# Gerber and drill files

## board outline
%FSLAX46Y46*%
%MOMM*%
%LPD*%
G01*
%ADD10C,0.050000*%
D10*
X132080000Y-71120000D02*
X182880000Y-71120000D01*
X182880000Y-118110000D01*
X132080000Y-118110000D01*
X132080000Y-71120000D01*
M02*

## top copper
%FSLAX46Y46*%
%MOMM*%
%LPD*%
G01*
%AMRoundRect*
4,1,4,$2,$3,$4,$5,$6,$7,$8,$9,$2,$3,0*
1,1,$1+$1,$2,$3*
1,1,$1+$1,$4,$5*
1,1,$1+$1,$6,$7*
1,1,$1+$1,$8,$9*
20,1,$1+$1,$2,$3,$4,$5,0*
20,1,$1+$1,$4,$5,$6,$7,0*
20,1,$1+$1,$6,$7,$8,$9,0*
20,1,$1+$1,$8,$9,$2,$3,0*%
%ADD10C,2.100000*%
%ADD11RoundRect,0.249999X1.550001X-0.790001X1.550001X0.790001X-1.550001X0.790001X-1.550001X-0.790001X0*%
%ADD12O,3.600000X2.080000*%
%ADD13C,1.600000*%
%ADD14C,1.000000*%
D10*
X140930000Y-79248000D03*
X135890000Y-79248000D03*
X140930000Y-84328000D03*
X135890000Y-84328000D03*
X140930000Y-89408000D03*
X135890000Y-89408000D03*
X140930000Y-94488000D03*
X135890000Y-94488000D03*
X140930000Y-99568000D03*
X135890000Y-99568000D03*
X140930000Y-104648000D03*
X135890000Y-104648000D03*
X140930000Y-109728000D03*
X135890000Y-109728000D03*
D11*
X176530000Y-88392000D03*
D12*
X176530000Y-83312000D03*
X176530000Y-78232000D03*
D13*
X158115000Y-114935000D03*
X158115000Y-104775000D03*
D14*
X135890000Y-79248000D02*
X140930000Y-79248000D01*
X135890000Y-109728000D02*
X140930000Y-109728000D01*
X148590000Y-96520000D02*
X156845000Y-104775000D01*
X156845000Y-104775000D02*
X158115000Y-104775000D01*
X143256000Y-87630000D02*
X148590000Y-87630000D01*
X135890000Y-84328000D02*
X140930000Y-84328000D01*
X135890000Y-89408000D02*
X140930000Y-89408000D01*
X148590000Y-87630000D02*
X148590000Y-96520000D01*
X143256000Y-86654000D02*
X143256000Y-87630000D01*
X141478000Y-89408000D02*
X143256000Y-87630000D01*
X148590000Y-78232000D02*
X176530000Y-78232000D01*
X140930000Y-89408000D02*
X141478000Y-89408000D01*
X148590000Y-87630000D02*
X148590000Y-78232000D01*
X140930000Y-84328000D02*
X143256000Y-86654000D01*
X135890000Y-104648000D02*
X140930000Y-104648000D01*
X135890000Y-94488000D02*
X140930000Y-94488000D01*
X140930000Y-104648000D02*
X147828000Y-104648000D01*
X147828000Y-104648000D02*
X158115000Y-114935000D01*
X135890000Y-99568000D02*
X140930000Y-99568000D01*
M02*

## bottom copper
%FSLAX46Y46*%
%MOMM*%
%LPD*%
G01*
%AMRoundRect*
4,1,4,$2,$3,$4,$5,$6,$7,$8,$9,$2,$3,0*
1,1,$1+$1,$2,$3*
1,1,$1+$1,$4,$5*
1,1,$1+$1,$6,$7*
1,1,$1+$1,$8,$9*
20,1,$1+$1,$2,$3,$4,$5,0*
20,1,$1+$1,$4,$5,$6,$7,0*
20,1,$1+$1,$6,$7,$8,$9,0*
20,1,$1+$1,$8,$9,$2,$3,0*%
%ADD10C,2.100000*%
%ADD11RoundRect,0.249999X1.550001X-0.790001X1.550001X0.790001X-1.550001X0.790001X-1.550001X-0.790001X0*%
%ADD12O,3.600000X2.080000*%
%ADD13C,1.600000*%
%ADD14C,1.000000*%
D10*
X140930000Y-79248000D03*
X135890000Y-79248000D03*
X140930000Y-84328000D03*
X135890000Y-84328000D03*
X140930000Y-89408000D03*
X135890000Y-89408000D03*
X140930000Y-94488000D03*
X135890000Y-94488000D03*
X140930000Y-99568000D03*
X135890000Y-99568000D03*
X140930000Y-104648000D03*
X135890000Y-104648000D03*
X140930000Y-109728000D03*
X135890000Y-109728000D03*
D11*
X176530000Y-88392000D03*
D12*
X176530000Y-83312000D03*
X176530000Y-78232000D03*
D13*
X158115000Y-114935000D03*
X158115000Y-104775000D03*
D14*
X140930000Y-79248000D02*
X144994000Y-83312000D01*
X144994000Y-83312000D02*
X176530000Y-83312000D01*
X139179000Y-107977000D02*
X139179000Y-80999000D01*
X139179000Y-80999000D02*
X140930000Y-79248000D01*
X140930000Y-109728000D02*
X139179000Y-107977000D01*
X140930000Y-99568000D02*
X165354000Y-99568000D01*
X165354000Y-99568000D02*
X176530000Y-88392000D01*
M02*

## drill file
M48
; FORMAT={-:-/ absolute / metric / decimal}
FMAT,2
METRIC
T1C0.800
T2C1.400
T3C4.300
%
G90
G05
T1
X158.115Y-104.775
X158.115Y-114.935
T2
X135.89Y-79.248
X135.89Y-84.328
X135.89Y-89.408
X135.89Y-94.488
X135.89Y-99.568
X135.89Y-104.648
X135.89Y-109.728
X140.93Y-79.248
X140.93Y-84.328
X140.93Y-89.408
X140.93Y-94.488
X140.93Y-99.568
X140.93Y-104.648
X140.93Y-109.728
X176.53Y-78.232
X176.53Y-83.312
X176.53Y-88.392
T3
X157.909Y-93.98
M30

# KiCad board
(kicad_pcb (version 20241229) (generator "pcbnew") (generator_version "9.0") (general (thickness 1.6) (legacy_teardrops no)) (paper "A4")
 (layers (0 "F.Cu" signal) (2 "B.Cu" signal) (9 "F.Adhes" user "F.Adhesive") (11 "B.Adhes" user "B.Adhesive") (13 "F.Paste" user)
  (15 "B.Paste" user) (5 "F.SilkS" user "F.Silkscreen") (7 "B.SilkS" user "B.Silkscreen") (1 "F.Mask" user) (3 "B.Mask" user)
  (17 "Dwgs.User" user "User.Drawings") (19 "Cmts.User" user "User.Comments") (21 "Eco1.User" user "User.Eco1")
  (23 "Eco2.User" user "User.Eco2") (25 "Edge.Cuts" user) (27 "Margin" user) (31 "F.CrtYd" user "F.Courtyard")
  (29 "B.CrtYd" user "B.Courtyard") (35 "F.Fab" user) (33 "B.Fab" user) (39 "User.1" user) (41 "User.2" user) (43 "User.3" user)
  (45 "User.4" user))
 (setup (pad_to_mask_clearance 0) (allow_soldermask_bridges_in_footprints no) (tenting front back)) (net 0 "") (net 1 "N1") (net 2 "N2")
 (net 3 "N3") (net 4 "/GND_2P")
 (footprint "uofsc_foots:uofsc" (layer "F.Cu") (at 174.498 108.204)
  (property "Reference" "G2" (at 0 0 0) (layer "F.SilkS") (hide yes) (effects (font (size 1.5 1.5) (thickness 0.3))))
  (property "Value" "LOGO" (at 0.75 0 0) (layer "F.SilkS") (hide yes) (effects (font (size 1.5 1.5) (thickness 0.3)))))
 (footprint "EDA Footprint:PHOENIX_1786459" (layer "F.Cu") (at 124.76 75.708 -90)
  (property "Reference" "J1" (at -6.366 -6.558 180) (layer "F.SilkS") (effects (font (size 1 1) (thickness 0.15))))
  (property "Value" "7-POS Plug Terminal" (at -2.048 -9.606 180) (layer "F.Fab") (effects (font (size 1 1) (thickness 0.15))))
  (pad "1" thru_hole circle (at 3.54 -16.17 270) (size 2.1 2.1) (drill 1.4) (layers "*.Cu" "*.Mask") (remove_unused_layers no) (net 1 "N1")
   (solder_mask_margin 0.102))
  (pad "1" thru_hole circle (at 3.54 -11.13 270) (size 2.1 2.1) (drill 1.4) (layers "*.Cu" "*.Mask") (remove_unused_layers no) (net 1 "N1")
   (solder_mask_margin 0.102))
  (pad "2" thru_hole circle (at 8.62 -16.17 270) (size 2.1 2.1) (drill 1.4) (layers "*.Cu" "*.Mask") (remove_unused_layers no) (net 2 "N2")
   (solder_mask_margin 0.102))
  (pad "2" thru_hole circle (at 8.62 -11.13 270) (size 2.1 2.1) (drill 1.4) (layers "*.Cu" "*.Mask") (remove_unused_layers no) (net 2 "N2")
   (solder_mask_margin 0.102))
  (pad "3" thru_hole circle (at 13.7 -16.17 270) (size 2.1 2.1) (drill 1.4) (layers "*.Cu" "*.Mask") (remove_unused_layers no) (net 2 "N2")
   (solder_mask_margin 0.102))
  (pad "3" thru_hole circle (at 13.7 -11.13 270) (size 2.1 2.1) (drill 1.4) (layers "*.Cu" "*.Mask") (remove_unused_layers no) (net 2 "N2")
   (solder_mask_margin 0.102))
  (pad "4" thru_hole circle (at 18.78 -16.17 270) (size 2.1 2.1) (drill 1.4) (layers "*.Cu" "*.Mask") (remove_unused_layers no) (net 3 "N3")
   (solder_mask_margin 0.102))
  (pad "4" thru_hole circle (at 18.78 -11.13 270) (size 2.1 2.1) (drill 1.4) (layers "*.Cu" "*.Mask") (remove_unused_layers no) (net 3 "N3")
   (solder_mask_margin 0.102))
  (pad "5" thru_hole circle (at 23.86 -16.17 270) (size 2.1 2.1) (drill 1.4) (layers "*.Cu" "*.Mask") (remove_unused_layers no)
   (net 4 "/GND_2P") (solder_mask_margin 0.102))
  (pad "5" thru_hole circle (at 23.86 -11.13 270) (size 2.1 2.1) (drill 1.4) (layers "*.Cu" "*.Mask") (remove_unused_layers no)
   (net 4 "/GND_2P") (solder_mask_margin 0.102))
  (pad "6" thru_hole circle (at 28.94 -16.17 270) (size 2.1 2.1) (drill 1.4) (layers "*.Cu" "*.Mask") (remove_unused_layers no) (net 3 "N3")
   (solder_mask_margin 0.102))
  (pad "6" thru_hole circle (at 28.94 -11.13 270) (size 2.1 2.1) (drill 1.4) (layers "*.Cu" "*.Mask") (remove_unused_layers no) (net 3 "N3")
   (solder_mask_margin 0.102))
  (pad "7" thru_hole circle (at 34.02 -16.17 270) (size 2.1 2.1) (drill 1.4) (layers "*.Cu" "*.Mask") (remove_unused_layers no) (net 1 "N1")
   (solder_mask_margin 0.102))
  (pad "7" thru_hole circle (at 34.02 -11.13 270) (size 2.1 2.1) (drill 1.4) (layers "*.Cu" "*.Mask") (remove_unused_layers no) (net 1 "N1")
   (solder_mask_margin 0.102)))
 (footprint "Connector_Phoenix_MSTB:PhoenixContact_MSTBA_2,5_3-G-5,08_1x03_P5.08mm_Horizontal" (layer "F.Cu") (at 176.53 88.392 90)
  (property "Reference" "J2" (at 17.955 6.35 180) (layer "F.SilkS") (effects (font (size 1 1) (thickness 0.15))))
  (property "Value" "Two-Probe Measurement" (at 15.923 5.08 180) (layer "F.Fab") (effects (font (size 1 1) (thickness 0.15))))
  (pad "1" thru_hole roundrect (at 0 0 90) (size 2.08 3.6) (drill 1.4) (layers "*.Cu" "*.Mask") (remove_unused_layers no)
   (roundrect_rratio 0.120192) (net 4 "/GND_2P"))
  (pad "2" thru_hole oval (at 5.08 0 90) (size 2.08 3.6) (drill 1.4) (layers "*.Cu" "*.Mask") (remove_unused_layers no) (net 1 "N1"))
  (pad "3" thru_hole oval (at 10.16 0 90) (size 2.08 3.6) (drill 1.4) (layers "*.Cu" "*.Mask") (remove_unused_layers no) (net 2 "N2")))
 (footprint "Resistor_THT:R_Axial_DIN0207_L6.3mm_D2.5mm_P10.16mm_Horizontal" (layer "F.Cu") (at 158.115 114.935 90)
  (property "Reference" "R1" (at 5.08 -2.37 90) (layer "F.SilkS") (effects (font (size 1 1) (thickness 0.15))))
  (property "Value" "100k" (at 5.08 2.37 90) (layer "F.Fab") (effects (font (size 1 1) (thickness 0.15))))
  (pad "1" thru_hole circle (at 0 0 90) (size 1.6 1.6) (drill 0.8) (layers "*.Cu" "*.Mask") (remove_unused_layers no) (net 3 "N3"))
  (pad "2" thru_hole circle (at 10.16 0 90) (size 1.6 1.6) (drill 0.8) (layers "*.Cu" "*.Mask") (remove_unused_layers no) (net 2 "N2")))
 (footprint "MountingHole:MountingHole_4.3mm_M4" (layer "F.Cu") (at 157.908508 93.98)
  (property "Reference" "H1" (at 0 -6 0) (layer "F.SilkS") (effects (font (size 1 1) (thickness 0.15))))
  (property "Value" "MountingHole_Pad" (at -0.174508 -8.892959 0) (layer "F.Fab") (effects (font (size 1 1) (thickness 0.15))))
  (pad "" np_thru_hole circle (at 0 0) (size 4.3 4.3) (drill 4.3) (layers "*.Cu" "*.Mask")))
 (gr_rect (start 132.08 71.12) (end 182.88 118.11) (stroke (width 0.05) (type default)) (fill no) (layer "Edge.Cuts"))
 (segment (start 135.89 79.248) (end 140.93 79.248) (width 1) (layer "F.Cu") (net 1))
 (segment (start 135.89 109.728) (end 140.93 109.728) (width 1) (layer "F.Cu") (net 1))
 (segment (start 140.93 79.248) (end 144.994 83.312) (width 1) (layer "B.Cu") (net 1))
 (segment (start 144.994 83.312) (end 176.53 83.312) (width 1) (layer "B.Cu") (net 1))
 (segment (start 139.179 107.977) (end 139.179 80.999) (width 1) (layer "B.Cu") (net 1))
 (segment (start 139.179 80.999) (end 140.93 79.248) (width 1) (layer "B.Cu") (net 1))
 (segment (start 140.93 109.728) (end 139.179 107.977) (width 1) (layer "B.Cu") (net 1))
 (segment (start 148.59 96.52) (end 156.845 104.775) (width 1) (layer "F.Cu") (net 2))
 (segment (start 156.845 104.775) (end 158.115 104.775) (width 1) (layer "F.Cu") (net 2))
 (segment (start 143.256 87.63) (end 148.59 87.63) (width 1) (layer "F.Cu") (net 2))
 (segment (start 135.89 84.328) (end 140.93 84.328) (width 1) (layer "F.Cu") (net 2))
 (segment (start 135.89 89.408) (end 140.93 89.408) (width 1) (layer "F.Cu") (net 2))
 (segment (start 148.59 87.63) (end 148.59 96.52) (width 1) (layer "F.Cu") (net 2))
 (segment (start 143.256 86.654) (end 143.256 87.63) (width 1) (layer "F.Cu") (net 2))
 (segment (start 141.478 89.408) (end 143.256 87.63) (width 1) (layer "F.Cu") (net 2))
 (segment (start 148.59 78.232) (end 176.53 78.232) (width 1) (layer "F.Cu") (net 2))
 (segment (start 140.93 89.408) (end 141.478 89.408) (width 1) (layer "F.Cu") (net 2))
 (segment (start 148.59 87.63) (end 148.59 78.232) (width 1) (layer "F.Cu") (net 2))
 (segment (start 140.93 84.328) (end 143.256 86.654) (width 1) (layer "F.Cu") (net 2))
 (segment (start 135.89 104.648) (end 140.93 104.648) (width 1) (layer "F.Cu") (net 3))
 (segment (start 135.89 94.488) (end 140.93 94.488) (width 1) (layer "F.Cu") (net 3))
 (segment (start 140.93 104.648) (end 147.828 104.648) (width 1) (layer "F.Cu") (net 3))
 (segment (start 147.828 104.648) (end 158.115 114.935) (width 1) (layer "F.Cu") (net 3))
 (segment (start 135.89 99.568) (end 140.93 99.568) (width 1) (layer "F.Cu") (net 4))
 (segment (start 140.93 99.568) (end 165.354 99.568) (width 1) (layer "B.Cu") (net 4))
 (segment (start 165.354 99.568) (end 176.53 88.392) (width 1) (layer "B.Cu") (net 4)))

